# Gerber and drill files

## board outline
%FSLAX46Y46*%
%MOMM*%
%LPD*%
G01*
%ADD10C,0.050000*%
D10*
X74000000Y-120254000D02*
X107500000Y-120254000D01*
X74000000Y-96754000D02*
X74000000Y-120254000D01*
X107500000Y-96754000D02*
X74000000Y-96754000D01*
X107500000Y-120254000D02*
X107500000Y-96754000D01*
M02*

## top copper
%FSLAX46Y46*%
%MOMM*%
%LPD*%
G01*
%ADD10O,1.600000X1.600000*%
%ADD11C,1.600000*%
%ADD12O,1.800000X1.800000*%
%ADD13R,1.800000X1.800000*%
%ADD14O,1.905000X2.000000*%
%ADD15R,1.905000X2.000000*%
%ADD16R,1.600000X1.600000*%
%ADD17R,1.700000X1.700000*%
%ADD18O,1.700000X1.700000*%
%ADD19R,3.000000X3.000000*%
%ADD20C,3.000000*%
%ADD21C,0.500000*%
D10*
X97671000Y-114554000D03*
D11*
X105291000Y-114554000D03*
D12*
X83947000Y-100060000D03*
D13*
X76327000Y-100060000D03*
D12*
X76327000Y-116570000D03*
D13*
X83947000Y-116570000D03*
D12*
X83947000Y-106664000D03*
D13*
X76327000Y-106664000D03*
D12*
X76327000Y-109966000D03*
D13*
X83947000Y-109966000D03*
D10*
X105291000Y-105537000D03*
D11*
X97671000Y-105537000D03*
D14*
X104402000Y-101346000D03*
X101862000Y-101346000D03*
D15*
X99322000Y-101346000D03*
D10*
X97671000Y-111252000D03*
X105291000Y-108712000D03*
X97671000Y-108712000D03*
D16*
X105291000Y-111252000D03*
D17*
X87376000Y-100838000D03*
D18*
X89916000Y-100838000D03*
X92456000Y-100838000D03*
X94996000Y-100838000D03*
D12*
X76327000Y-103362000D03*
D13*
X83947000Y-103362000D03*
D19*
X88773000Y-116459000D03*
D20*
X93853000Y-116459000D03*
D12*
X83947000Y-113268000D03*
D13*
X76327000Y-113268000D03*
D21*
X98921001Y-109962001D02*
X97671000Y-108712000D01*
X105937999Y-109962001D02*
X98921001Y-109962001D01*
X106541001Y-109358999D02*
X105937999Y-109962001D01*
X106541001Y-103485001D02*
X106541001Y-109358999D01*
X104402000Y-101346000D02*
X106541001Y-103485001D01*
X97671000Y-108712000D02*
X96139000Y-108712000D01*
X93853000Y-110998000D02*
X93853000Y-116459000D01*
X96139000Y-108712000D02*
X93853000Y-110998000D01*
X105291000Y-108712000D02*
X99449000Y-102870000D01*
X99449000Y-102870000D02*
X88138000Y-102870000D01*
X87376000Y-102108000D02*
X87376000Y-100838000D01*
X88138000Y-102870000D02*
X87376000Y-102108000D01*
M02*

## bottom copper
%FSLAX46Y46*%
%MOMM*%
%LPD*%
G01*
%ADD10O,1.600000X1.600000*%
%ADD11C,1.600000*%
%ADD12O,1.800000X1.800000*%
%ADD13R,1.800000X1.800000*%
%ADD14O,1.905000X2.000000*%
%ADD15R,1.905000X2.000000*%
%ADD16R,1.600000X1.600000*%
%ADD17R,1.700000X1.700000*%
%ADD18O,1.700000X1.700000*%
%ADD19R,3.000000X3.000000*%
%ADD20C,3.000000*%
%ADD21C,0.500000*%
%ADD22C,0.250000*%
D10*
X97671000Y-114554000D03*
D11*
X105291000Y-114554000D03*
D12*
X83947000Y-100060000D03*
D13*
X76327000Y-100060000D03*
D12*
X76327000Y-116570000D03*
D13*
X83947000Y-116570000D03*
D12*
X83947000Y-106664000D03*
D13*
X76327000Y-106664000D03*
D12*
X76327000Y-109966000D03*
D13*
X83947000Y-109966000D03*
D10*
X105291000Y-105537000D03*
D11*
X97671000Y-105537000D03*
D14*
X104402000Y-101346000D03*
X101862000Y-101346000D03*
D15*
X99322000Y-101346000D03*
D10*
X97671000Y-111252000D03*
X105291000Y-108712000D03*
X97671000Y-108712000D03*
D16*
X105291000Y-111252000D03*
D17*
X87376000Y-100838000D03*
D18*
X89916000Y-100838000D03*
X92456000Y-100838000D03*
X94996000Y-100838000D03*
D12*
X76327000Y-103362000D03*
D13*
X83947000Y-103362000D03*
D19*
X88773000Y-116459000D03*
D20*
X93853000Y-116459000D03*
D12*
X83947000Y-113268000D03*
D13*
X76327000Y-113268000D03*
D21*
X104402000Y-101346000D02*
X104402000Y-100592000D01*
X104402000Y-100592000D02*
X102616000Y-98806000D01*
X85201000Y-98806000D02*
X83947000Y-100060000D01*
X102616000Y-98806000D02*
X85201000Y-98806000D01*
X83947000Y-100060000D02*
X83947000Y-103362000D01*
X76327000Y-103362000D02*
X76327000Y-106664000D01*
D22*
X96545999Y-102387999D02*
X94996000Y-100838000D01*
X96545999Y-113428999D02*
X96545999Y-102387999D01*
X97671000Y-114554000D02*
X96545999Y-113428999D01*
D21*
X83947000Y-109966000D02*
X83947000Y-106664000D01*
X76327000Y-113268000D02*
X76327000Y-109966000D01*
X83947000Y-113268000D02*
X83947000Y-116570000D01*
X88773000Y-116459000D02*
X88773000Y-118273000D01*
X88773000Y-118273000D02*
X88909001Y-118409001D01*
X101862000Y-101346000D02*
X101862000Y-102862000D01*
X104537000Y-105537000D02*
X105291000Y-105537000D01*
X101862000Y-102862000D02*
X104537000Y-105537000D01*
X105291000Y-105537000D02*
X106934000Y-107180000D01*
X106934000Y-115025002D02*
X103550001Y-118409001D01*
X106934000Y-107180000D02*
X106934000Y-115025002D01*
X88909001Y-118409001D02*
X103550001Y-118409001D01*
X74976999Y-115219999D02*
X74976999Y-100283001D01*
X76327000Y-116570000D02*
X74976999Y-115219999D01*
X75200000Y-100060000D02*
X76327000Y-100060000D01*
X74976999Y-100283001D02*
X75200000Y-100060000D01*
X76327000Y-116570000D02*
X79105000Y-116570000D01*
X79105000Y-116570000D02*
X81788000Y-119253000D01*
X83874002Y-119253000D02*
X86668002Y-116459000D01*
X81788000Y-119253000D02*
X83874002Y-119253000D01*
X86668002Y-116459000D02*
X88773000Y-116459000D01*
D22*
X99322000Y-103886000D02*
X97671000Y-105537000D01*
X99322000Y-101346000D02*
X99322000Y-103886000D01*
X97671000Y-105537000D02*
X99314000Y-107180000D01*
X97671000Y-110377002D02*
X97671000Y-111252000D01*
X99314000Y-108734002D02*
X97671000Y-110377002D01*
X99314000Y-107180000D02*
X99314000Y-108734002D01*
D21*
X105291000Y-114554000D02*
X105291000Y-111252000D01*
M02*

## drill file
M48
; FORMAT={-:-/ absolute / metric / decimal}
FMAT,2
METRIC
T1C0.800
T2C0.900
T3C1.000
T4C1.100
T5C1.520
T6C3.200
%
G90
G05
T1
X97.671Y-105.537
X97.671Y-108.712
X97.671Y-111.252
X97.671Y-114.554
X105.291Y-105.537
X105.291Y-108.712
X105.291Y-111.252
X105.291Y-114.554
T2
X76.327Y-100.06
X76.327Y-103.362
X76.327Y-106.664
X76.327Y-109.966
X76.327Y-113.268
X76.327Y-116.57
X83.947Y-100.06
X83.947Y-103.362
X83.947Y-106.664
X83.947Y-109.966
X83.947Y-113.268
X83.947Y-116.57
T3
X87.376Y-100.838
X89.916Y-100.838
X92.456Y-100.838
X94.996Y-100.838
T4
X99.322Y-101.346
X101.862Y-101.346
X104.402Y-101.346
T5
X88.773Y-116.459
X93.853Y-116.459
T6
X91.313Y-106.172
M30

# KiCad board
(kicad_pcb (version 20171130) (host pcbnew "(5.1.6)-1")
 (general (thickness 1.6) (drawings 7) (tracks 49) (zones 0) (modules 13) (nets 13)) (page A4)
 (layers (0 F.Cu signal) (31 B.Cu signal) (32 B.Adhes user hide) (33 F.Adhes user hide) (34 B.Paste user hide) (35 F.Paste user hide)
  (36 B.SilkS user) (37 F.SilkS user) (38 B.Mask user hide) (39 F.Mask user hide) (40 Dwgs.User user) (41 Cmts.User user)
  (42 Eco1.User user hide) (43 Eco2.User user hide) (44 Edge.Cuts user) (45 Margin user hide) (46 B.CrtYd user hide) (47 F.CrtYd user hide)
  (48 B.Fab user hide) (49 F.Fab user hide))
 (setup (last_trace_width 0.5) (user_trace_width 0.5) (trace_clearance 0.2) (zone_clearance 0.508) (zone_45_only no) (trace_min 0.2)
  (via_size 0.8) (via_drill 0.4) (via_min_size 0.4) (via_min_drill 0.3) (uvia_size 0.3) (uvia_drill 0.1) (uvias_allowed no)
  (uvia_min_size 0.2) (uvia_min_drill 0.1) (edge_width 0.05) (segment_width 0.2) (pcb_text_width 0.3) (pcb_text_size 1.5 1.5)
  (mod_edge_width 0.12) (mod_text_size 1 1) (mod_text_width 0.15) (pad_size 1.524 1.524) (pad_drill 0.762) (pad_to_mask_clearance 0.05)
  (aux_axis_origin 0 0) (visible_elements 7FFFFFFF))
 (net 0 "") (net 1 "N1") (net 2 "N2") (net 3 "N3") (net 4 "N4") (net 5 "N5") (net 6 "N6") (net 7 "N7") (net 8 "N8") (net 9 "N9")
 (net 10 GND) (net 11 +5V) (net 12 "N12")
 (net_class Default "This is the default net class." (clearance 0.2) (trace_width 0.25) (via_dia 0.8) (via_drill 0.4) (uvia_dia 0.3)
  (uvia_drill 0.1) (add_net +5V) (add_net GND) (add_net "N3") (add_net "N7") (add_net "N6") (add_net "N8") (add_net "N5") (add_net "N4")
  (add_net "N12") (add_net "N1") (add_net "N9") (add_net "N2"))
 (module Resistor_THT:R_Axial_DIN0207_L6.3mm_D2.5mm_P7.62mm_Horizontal (layer F.Cu) (at 105.291 114.554 180)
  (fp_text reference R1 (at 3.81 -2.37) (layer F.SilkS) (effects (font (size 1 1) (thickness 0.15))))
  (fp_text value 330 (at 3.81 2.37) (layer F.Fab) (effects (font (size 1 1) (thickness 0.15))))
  (pad 2 thru_hole oval (at 7.62 0 180) (size 1.6 1.6) (drill 0.8) (layers *.Cu *.Mask) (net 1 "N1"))
  (pad 1 thru_hole circle (at 0 0 180) (size 1.6 1.6) (drill 0.8) (layers *.Cu *.Mask) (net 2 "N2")))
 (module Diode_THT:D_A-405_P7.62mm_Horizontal (layer F.Cu) (at 76.327 100.06)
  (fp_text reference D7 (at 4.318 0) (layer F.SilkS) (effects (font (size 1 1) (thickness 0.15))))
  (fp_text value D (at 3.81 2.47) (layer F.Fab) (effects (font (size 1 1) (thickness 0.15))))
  (pad 2 thru_hole oval (at 7.62 0) (size 1.8 1.8) (drill 0.9) (layers *.Cu *.Mask) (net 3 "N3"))
  (pad 1 thru_hole rect (at 0 0) (size 1.8 1.8) (drill 0.9) (layers *.Cu *.Mask) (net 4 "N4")))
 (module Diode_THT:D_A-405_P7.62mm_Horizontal (layer F.Cu) (at 83.947 116.57 180)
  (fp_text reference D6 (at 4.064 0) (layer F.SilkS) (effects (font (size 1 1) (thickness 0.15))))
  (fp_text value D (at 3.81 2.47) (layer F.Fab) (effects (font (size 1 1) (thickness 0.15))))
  (pad 2 thru_hole oval (at 7.62 0 180) (size 1.8 1.8) (drill 0.9) (layers *.Cu *.Mask) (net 4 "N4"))
  (pad 1 thru_hole rect (at 0 0 180) (size 1.8 1.8) (drill 0.9) (layers *.Cu *.Mask) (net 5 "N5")))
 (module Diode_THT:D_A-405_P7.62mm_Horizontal (layer F.Cu) (at 76.327 106.664)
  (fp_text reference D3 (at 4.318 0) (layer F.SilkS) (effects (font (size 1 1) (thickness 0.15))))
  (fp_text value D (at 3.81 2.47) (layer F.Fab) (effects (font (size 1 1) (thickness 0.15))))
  (pad 2 thru_hole oval (at 7.62 0) (size 1.8 1.8) (drill 0.9) (layers *.Cu *.Mask) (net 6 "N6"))
  (pad 1 thru_hole rect (at 0 0) (size 1.8 1.8) (drill 0.9) (layers *.Cu *.Mask) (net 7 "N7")))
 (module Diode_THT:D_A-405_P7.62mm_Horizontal (layer F.Cu) (at 83.947 109.966 180)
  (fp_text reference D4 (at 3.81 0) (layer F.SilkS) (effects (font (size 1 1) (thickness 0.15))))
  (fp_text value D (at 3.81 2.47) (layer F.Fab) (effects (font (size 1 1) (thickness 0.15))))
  (pad 2 thru_hole oval (at 7.62 0 180) (size 1.8 1.8) (drill 0.9) (layers *.Cu *.Mask) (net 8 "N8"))
  (pad 1 thru_hole rect (at 0 0 180) (size 1.8 1.8) (drill 0.9) (layers *.Cu *.Mask) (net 6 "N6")))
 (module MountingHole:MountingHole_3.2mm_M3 (layer F.Cu) (at 91.313 106.172)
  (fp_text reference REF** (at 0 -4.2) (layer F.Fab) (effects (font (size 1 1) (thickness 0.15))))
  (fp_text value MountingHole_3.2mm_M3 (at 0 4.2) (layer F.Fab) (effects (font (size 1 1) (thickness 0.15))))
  (pad 1 np_thru_hole circle (at 0 0) (size 3.2 3.2) (drill 3.2) (layers *.Cu *.Mask)))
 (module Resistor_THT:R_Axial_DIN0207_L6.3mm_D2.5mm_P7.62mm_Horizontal (layer F.Cu) (at 97.671 105.537)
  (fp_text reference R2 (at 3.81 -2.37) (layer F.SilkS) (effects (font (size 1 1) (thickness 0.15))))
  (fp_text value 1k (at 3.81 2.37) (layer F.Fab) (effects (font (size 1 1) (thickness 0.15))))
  (pad 2 thru_hole oval (at 7.62 0) (size 1.6 1.6) (drill 0.8) (layers *.Cu *.Mask) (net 4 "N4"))
  (pad 1 thru_hole circle (at 0 0) (size 1.6 1.6) (drill 0.8) (layers *.Cu *.Mask) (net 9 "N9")))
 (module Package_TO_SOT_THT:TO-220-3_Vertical (layer F.Cu) (at 99.322 101.346)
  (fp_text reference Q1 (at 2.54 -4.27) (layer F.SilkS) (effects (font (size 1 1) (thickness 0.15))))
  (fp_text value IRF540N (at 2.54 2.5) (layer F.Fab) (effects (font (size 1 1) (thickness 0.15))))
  (pad 3 thru_hole oval (at 5.08 0) (size 1.905 2) (drill 1.1) (layers *.Cu *.Mask) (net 3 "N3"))
  (pad 2 thru_hole oval (at 2.54 0) (size 1.905 2) (drill 1.1) (layers *.Cu *.Mask) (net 4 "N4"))
  (pad 1 thru_hole rect (at 0 0) (size 1.905 2) (drill 1.1) (layers *.Cu *.Mask) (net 9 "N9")))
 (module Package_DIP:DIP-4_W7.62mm (layer F.Cu) (at 105.291 111.252 180)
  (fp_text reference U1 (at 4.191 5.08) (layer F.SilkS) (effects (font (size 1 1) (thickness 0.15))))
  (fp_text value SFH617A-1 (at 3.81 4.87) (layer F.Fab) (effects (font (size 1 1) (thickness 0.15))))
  (pad 4 thru_hole oval (at 7.62 0 180) (size 1.6 1.6) (drill 0.8) (layers *.Cu *.Mask) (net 9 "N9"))
  (pad 2 thru_hole oval (at 0 2.54 180) (size 1.6 1.6) (drill 0.8) (layers *.Cu *.Mask) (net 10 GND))
  (pad 3 thru_hole oval (at 7.62 2.54 180) (size 1.6 1.6) (drill 0.8) (layers *.Cu *.Mask) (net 3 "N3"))
  (pad 1 thru_hole rect (at 0 0 180) (size 1.6 1.6) (drill 0.8) (layers *.Cu *.Mask) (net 2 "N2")))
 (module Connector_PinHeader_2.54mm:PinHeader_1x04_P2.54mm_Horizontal (layer F.Cu) (at 87.376 100.838 90)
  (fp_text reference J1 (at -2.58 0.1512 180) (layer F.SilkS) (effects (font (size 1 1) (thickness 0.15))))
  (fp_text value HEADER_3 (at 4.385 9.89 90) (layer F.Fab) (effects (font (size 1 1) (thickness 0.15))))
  (pad 1 thru_hole rect (at 0 0 90) (size 1.7 1.7) (drill 1) (layers *.Cu *.Mask) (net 10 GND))
  (pad 2 thru_hole oval (at 0 2.54 90) (size 1.7 1.7) (drill 1) (layers *.Cu *.Mask) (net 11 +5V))
  (pad 3 thru_hole oval (at 0 5.08 90) (size 1.7 1.7) (drill 1) (layers *.Cu *.Mask) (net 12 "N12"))
  (pad 4 thru_hole oval (at 0 7.62 90) (size 1.7 1.7) (drill 1) (layers *.Cu *.Mask) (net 1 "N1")))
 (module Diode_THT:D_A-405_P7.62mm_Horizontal (layer F.Cu) (at 83.947 103.362 180)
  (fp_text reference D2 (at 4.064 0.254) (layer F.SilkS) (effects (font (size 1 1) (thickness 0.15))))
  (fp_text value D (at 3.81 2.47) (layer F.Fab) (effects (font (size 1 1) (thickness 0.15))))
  (pad 2 thru_hole oval (at 7.62 0 180) (size 1.8 1.8) (drill 0.9) (layers *.Cu *.Mask) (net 7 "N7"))
  (pad 1 thru_hole rect (at 0 0 180) (size 1.8 1.8) (drill 0.9) (layers *.Cu *.Mask) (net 3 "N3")))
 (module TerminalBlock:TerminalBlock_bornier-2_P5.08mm (layer F.Cu) (at 88.773 116.459)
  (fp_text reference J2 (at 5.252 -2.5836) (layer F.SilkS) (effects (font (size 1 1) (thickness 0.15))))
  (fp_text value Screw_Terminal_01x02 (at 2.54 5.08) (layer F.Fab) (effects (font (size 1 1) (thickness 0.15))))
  (pad 1 thru_hole rect (at 0 0) (size 3 3) (drill 1.52) (layers *.Cu *.Mask) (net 4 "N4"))
  (pad 2 thru_hole circle (at 5.08 0) (size 3 3) (drill 1.52) (layers *.Cu *.Mask) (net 3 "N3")))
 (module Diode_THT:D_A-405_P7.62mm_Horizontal (layer F.Cu) (at 76.327 113.268)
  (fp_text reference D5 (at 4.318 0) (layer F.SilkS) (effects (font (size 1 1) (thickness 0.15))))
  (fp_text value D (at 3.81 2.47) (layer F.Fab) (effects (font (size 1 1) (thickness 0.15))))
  (pad 2 thru_hole oval (at 7.62 0) (size 1.8 1.8) (drill 0.9) (layers *.Cu *.Mask) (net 5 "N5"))
  (pad 1 thru_hole rect (at 0 0) (size 1.8 1.8) (drill 0.9) (layers *.Cu *.Mask) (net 8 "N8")))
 (gr_line (start 74 120.254) (end 107.5 120.254) (layer Edge.Cuts) (width 0.05))
 (gr_line (start 74 96.754) (end 74 120.254) (layer Edge.Cuts) (width 0.05))
 (gr_line (start 107.5 96.754) (end 74 96.754) (layer Edge.Cuts) (width 0.05))
 (gr_line (start 107.5 120.254) (end 107.5 96.754) (layer Edge.Cuts) (width 0.05))
 (segment (start 104.402 101.346) (end 104.402 100.592) (width 0.5) (layer B.Cu) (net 3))
 (segment (start 104.402 100.592) (end 102.616 98.806) (width 0.5) (layer B.Cu) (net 3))
 (segment (start 85.201 98.806) (end 83.947 100.06) (width 0.5) (layer B.Cu) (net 3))
 (segment (start 102.616 98.806) (end 85.201 98.806) (width 0.5) (layer B.Cu) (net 3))
 (segment (start 83.947 100.06) (end 83.947 103.362) (width 0.5) (layer B.Cu) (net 3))
 (segment (start 98.921001 109.962001) (end 97.671 108.712) (width 0.5) (layer F.Cu) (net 3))
 (segment (start 105.937999 109.962001) (end 98.921001 109.962001) (width 0.5) (layer F.Cu) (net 3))
 (segment (start 106.541001 109.358999) (end 105.937999 109.962001) (width 0.5) (layer F.Cu) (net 3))
 (segment (start 106.541001 103.485001) (end 106.541001 109.358999) (width 0.5) (layer F.Cu) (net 3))
 (segment (start 104.402 101.346) (end 106.541001 103.485001) (width 0.5) (layer F.Cu) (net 3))
 (segment (start 97.671 108.712) (end 96.139 108.712) (width 0.5) (layer F.Cu) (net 3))
 (segment (start 93.853 110.998) (end 93.853 116.459) (width 0.5) (layer F.Cu) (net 3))
 (segment (start 96.139 108.712) (end 93.853 110.998) (width 0.5) (layer F.Cu) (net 3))
 (segment (start 76.327 103.362) (end 76.327 106.664) (width 0.5) (layer B.Cu) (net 7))
 (segment (start 96.545999 102.387999) (end 94.996 100.838) (width 0.25) (layer B.Cu) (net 1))
 (segment (start 96.545999 113.428999) (end 96.545999 102.387999) (width 0.25) (layer B.Cu) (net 1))
 (segment (start 97.671 114.554) (end 96.545999 113.428999) (width 0.25) (layer B.Cu) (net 1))
 (segment (start 105.291 108.712) (end 99.449 102.87) (width 0.5) (layer F.Cu) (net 10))
 (segment (start 99.449 102.87) (end 88.138 102.87) (width 0.5) (layer F.Cu) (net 10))
 (segment (start 87.376 102.108) (end 87.376 100.838) (width 0.5) (layer F.Cu) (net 10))
 (segment (start 88.138 102.87) (end 87.376 102.108) (width 0.5) (layer F.Cu) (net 10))
 (segment (start 83.947 109.966) (end 83.947 106.664) (width 0.5) (layer B.Cu) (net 6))
 (segment (start 76.327 113.268) (end 76.327 109.966) (width 0.5) (layer B.Cu) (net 8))
 (segment (start 83.947 113.268) (end 83.947 116.57) (width 0.5) (layer B.Cu) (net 5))
 (segment (start 88.773 116.459) (end 88.773 118.273) (width 0.5) (layer B.Cu) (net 4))
 (segment (start 88.773 118.273) (end 88.909001 118.409001) (width 0.5) (layer B.Cu) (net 4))
 (segment (start 101.862 101.346) (end 101.862 102.862) (width 0.5) (layer B.Cu) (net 4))
 (segment (start 104.537 105.537) (end 105.291 105.537) (width 0.5) (layer B.Cu) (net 4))
 (segment (start 101.862 102.862) (end 104.537 105.537) (width 0.5) (layer B.Cu) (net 4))
 (segment (start 105.291 105.537) (end 106.934 107.18) (width 0.5) (layer B.Cu) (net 4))
 (segment (start 106.934 115.025002) (end 103.550001 118.409001) (width 0.5) (layer B.Cu) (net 4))
 (segment (start 106.934 107.18) (end 106.934 115.025002) (width 0.5) (layer B.Cu) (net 4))
 (segment (start 88.909001 118.409001) (end 103.550001 118.409001) (width 0.5) (layer B.Cu) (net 4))
 (segment (start 74.976999 115.219999) (end 74.976999 100.283001) (width 0.5) (layer B.Cu) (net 4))
 (segment (start 76.327 116.57) (end 74.976999 115.219999) (width 0.5) (layer B.Cu) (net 4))
 (segment (start 75.2 100.06) (end 76.327 100.06) (width 0.5) (layer B.Cu) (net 4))
 (segment (start 74.976999 100.283001) (end 75.2 100.06) (width 0.5) (layer B.Cu) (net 4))
 (segment (start 76.327 116.57) (end 79.105 116.57) (width 0.5) (layer B.Cu) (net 4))
 (segment (start 79.105 116.57) (end 81.788 119.253) (width 0.5) (layer B.Cu) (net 4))
 (segment (start 83.874002 119.253) (end 86.668002 116.459) (width 0.5) (layer B.Cu) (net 4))
 (segment (start 81.788 119.253) (end 83.874002 119.253) (width 0.5) (layer B.Cu) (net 4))
 (segment (start 86.668002 116.459) (end 88.773 116.459) (width 0.5) (layer B.Cu) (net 4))
 (segment (start 99.322 103.886) (end 97.671 105.537) (width 0.25) (layer B.Cu) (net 9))
 (segment (start 99.322 101.346) (end 99.322 103.886) (width 0.25) (layer B.Cu) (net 9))
 (segment (start 97.671 105.537) (end 99.314 107.18) (width 0.25) (layer B.Cu) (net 9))
 (segment (start 97.671 110.377002) (end 97.671 111.252) (width 0.25) (layer B.Cu) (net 9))
 (segment (start 99.314 108.734002) (end 97.671 110.377002) (width 0.25) (layer B.Cu) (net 9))
 (segment (start 99.314 107.18) (end 99.314 108.734002) (width 0.25) (layer B.Cu) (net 9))
 (segment (start 105.291 114.554) (end 105.291 111.252) (width 0.5) (layer B.Cu) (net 2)))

